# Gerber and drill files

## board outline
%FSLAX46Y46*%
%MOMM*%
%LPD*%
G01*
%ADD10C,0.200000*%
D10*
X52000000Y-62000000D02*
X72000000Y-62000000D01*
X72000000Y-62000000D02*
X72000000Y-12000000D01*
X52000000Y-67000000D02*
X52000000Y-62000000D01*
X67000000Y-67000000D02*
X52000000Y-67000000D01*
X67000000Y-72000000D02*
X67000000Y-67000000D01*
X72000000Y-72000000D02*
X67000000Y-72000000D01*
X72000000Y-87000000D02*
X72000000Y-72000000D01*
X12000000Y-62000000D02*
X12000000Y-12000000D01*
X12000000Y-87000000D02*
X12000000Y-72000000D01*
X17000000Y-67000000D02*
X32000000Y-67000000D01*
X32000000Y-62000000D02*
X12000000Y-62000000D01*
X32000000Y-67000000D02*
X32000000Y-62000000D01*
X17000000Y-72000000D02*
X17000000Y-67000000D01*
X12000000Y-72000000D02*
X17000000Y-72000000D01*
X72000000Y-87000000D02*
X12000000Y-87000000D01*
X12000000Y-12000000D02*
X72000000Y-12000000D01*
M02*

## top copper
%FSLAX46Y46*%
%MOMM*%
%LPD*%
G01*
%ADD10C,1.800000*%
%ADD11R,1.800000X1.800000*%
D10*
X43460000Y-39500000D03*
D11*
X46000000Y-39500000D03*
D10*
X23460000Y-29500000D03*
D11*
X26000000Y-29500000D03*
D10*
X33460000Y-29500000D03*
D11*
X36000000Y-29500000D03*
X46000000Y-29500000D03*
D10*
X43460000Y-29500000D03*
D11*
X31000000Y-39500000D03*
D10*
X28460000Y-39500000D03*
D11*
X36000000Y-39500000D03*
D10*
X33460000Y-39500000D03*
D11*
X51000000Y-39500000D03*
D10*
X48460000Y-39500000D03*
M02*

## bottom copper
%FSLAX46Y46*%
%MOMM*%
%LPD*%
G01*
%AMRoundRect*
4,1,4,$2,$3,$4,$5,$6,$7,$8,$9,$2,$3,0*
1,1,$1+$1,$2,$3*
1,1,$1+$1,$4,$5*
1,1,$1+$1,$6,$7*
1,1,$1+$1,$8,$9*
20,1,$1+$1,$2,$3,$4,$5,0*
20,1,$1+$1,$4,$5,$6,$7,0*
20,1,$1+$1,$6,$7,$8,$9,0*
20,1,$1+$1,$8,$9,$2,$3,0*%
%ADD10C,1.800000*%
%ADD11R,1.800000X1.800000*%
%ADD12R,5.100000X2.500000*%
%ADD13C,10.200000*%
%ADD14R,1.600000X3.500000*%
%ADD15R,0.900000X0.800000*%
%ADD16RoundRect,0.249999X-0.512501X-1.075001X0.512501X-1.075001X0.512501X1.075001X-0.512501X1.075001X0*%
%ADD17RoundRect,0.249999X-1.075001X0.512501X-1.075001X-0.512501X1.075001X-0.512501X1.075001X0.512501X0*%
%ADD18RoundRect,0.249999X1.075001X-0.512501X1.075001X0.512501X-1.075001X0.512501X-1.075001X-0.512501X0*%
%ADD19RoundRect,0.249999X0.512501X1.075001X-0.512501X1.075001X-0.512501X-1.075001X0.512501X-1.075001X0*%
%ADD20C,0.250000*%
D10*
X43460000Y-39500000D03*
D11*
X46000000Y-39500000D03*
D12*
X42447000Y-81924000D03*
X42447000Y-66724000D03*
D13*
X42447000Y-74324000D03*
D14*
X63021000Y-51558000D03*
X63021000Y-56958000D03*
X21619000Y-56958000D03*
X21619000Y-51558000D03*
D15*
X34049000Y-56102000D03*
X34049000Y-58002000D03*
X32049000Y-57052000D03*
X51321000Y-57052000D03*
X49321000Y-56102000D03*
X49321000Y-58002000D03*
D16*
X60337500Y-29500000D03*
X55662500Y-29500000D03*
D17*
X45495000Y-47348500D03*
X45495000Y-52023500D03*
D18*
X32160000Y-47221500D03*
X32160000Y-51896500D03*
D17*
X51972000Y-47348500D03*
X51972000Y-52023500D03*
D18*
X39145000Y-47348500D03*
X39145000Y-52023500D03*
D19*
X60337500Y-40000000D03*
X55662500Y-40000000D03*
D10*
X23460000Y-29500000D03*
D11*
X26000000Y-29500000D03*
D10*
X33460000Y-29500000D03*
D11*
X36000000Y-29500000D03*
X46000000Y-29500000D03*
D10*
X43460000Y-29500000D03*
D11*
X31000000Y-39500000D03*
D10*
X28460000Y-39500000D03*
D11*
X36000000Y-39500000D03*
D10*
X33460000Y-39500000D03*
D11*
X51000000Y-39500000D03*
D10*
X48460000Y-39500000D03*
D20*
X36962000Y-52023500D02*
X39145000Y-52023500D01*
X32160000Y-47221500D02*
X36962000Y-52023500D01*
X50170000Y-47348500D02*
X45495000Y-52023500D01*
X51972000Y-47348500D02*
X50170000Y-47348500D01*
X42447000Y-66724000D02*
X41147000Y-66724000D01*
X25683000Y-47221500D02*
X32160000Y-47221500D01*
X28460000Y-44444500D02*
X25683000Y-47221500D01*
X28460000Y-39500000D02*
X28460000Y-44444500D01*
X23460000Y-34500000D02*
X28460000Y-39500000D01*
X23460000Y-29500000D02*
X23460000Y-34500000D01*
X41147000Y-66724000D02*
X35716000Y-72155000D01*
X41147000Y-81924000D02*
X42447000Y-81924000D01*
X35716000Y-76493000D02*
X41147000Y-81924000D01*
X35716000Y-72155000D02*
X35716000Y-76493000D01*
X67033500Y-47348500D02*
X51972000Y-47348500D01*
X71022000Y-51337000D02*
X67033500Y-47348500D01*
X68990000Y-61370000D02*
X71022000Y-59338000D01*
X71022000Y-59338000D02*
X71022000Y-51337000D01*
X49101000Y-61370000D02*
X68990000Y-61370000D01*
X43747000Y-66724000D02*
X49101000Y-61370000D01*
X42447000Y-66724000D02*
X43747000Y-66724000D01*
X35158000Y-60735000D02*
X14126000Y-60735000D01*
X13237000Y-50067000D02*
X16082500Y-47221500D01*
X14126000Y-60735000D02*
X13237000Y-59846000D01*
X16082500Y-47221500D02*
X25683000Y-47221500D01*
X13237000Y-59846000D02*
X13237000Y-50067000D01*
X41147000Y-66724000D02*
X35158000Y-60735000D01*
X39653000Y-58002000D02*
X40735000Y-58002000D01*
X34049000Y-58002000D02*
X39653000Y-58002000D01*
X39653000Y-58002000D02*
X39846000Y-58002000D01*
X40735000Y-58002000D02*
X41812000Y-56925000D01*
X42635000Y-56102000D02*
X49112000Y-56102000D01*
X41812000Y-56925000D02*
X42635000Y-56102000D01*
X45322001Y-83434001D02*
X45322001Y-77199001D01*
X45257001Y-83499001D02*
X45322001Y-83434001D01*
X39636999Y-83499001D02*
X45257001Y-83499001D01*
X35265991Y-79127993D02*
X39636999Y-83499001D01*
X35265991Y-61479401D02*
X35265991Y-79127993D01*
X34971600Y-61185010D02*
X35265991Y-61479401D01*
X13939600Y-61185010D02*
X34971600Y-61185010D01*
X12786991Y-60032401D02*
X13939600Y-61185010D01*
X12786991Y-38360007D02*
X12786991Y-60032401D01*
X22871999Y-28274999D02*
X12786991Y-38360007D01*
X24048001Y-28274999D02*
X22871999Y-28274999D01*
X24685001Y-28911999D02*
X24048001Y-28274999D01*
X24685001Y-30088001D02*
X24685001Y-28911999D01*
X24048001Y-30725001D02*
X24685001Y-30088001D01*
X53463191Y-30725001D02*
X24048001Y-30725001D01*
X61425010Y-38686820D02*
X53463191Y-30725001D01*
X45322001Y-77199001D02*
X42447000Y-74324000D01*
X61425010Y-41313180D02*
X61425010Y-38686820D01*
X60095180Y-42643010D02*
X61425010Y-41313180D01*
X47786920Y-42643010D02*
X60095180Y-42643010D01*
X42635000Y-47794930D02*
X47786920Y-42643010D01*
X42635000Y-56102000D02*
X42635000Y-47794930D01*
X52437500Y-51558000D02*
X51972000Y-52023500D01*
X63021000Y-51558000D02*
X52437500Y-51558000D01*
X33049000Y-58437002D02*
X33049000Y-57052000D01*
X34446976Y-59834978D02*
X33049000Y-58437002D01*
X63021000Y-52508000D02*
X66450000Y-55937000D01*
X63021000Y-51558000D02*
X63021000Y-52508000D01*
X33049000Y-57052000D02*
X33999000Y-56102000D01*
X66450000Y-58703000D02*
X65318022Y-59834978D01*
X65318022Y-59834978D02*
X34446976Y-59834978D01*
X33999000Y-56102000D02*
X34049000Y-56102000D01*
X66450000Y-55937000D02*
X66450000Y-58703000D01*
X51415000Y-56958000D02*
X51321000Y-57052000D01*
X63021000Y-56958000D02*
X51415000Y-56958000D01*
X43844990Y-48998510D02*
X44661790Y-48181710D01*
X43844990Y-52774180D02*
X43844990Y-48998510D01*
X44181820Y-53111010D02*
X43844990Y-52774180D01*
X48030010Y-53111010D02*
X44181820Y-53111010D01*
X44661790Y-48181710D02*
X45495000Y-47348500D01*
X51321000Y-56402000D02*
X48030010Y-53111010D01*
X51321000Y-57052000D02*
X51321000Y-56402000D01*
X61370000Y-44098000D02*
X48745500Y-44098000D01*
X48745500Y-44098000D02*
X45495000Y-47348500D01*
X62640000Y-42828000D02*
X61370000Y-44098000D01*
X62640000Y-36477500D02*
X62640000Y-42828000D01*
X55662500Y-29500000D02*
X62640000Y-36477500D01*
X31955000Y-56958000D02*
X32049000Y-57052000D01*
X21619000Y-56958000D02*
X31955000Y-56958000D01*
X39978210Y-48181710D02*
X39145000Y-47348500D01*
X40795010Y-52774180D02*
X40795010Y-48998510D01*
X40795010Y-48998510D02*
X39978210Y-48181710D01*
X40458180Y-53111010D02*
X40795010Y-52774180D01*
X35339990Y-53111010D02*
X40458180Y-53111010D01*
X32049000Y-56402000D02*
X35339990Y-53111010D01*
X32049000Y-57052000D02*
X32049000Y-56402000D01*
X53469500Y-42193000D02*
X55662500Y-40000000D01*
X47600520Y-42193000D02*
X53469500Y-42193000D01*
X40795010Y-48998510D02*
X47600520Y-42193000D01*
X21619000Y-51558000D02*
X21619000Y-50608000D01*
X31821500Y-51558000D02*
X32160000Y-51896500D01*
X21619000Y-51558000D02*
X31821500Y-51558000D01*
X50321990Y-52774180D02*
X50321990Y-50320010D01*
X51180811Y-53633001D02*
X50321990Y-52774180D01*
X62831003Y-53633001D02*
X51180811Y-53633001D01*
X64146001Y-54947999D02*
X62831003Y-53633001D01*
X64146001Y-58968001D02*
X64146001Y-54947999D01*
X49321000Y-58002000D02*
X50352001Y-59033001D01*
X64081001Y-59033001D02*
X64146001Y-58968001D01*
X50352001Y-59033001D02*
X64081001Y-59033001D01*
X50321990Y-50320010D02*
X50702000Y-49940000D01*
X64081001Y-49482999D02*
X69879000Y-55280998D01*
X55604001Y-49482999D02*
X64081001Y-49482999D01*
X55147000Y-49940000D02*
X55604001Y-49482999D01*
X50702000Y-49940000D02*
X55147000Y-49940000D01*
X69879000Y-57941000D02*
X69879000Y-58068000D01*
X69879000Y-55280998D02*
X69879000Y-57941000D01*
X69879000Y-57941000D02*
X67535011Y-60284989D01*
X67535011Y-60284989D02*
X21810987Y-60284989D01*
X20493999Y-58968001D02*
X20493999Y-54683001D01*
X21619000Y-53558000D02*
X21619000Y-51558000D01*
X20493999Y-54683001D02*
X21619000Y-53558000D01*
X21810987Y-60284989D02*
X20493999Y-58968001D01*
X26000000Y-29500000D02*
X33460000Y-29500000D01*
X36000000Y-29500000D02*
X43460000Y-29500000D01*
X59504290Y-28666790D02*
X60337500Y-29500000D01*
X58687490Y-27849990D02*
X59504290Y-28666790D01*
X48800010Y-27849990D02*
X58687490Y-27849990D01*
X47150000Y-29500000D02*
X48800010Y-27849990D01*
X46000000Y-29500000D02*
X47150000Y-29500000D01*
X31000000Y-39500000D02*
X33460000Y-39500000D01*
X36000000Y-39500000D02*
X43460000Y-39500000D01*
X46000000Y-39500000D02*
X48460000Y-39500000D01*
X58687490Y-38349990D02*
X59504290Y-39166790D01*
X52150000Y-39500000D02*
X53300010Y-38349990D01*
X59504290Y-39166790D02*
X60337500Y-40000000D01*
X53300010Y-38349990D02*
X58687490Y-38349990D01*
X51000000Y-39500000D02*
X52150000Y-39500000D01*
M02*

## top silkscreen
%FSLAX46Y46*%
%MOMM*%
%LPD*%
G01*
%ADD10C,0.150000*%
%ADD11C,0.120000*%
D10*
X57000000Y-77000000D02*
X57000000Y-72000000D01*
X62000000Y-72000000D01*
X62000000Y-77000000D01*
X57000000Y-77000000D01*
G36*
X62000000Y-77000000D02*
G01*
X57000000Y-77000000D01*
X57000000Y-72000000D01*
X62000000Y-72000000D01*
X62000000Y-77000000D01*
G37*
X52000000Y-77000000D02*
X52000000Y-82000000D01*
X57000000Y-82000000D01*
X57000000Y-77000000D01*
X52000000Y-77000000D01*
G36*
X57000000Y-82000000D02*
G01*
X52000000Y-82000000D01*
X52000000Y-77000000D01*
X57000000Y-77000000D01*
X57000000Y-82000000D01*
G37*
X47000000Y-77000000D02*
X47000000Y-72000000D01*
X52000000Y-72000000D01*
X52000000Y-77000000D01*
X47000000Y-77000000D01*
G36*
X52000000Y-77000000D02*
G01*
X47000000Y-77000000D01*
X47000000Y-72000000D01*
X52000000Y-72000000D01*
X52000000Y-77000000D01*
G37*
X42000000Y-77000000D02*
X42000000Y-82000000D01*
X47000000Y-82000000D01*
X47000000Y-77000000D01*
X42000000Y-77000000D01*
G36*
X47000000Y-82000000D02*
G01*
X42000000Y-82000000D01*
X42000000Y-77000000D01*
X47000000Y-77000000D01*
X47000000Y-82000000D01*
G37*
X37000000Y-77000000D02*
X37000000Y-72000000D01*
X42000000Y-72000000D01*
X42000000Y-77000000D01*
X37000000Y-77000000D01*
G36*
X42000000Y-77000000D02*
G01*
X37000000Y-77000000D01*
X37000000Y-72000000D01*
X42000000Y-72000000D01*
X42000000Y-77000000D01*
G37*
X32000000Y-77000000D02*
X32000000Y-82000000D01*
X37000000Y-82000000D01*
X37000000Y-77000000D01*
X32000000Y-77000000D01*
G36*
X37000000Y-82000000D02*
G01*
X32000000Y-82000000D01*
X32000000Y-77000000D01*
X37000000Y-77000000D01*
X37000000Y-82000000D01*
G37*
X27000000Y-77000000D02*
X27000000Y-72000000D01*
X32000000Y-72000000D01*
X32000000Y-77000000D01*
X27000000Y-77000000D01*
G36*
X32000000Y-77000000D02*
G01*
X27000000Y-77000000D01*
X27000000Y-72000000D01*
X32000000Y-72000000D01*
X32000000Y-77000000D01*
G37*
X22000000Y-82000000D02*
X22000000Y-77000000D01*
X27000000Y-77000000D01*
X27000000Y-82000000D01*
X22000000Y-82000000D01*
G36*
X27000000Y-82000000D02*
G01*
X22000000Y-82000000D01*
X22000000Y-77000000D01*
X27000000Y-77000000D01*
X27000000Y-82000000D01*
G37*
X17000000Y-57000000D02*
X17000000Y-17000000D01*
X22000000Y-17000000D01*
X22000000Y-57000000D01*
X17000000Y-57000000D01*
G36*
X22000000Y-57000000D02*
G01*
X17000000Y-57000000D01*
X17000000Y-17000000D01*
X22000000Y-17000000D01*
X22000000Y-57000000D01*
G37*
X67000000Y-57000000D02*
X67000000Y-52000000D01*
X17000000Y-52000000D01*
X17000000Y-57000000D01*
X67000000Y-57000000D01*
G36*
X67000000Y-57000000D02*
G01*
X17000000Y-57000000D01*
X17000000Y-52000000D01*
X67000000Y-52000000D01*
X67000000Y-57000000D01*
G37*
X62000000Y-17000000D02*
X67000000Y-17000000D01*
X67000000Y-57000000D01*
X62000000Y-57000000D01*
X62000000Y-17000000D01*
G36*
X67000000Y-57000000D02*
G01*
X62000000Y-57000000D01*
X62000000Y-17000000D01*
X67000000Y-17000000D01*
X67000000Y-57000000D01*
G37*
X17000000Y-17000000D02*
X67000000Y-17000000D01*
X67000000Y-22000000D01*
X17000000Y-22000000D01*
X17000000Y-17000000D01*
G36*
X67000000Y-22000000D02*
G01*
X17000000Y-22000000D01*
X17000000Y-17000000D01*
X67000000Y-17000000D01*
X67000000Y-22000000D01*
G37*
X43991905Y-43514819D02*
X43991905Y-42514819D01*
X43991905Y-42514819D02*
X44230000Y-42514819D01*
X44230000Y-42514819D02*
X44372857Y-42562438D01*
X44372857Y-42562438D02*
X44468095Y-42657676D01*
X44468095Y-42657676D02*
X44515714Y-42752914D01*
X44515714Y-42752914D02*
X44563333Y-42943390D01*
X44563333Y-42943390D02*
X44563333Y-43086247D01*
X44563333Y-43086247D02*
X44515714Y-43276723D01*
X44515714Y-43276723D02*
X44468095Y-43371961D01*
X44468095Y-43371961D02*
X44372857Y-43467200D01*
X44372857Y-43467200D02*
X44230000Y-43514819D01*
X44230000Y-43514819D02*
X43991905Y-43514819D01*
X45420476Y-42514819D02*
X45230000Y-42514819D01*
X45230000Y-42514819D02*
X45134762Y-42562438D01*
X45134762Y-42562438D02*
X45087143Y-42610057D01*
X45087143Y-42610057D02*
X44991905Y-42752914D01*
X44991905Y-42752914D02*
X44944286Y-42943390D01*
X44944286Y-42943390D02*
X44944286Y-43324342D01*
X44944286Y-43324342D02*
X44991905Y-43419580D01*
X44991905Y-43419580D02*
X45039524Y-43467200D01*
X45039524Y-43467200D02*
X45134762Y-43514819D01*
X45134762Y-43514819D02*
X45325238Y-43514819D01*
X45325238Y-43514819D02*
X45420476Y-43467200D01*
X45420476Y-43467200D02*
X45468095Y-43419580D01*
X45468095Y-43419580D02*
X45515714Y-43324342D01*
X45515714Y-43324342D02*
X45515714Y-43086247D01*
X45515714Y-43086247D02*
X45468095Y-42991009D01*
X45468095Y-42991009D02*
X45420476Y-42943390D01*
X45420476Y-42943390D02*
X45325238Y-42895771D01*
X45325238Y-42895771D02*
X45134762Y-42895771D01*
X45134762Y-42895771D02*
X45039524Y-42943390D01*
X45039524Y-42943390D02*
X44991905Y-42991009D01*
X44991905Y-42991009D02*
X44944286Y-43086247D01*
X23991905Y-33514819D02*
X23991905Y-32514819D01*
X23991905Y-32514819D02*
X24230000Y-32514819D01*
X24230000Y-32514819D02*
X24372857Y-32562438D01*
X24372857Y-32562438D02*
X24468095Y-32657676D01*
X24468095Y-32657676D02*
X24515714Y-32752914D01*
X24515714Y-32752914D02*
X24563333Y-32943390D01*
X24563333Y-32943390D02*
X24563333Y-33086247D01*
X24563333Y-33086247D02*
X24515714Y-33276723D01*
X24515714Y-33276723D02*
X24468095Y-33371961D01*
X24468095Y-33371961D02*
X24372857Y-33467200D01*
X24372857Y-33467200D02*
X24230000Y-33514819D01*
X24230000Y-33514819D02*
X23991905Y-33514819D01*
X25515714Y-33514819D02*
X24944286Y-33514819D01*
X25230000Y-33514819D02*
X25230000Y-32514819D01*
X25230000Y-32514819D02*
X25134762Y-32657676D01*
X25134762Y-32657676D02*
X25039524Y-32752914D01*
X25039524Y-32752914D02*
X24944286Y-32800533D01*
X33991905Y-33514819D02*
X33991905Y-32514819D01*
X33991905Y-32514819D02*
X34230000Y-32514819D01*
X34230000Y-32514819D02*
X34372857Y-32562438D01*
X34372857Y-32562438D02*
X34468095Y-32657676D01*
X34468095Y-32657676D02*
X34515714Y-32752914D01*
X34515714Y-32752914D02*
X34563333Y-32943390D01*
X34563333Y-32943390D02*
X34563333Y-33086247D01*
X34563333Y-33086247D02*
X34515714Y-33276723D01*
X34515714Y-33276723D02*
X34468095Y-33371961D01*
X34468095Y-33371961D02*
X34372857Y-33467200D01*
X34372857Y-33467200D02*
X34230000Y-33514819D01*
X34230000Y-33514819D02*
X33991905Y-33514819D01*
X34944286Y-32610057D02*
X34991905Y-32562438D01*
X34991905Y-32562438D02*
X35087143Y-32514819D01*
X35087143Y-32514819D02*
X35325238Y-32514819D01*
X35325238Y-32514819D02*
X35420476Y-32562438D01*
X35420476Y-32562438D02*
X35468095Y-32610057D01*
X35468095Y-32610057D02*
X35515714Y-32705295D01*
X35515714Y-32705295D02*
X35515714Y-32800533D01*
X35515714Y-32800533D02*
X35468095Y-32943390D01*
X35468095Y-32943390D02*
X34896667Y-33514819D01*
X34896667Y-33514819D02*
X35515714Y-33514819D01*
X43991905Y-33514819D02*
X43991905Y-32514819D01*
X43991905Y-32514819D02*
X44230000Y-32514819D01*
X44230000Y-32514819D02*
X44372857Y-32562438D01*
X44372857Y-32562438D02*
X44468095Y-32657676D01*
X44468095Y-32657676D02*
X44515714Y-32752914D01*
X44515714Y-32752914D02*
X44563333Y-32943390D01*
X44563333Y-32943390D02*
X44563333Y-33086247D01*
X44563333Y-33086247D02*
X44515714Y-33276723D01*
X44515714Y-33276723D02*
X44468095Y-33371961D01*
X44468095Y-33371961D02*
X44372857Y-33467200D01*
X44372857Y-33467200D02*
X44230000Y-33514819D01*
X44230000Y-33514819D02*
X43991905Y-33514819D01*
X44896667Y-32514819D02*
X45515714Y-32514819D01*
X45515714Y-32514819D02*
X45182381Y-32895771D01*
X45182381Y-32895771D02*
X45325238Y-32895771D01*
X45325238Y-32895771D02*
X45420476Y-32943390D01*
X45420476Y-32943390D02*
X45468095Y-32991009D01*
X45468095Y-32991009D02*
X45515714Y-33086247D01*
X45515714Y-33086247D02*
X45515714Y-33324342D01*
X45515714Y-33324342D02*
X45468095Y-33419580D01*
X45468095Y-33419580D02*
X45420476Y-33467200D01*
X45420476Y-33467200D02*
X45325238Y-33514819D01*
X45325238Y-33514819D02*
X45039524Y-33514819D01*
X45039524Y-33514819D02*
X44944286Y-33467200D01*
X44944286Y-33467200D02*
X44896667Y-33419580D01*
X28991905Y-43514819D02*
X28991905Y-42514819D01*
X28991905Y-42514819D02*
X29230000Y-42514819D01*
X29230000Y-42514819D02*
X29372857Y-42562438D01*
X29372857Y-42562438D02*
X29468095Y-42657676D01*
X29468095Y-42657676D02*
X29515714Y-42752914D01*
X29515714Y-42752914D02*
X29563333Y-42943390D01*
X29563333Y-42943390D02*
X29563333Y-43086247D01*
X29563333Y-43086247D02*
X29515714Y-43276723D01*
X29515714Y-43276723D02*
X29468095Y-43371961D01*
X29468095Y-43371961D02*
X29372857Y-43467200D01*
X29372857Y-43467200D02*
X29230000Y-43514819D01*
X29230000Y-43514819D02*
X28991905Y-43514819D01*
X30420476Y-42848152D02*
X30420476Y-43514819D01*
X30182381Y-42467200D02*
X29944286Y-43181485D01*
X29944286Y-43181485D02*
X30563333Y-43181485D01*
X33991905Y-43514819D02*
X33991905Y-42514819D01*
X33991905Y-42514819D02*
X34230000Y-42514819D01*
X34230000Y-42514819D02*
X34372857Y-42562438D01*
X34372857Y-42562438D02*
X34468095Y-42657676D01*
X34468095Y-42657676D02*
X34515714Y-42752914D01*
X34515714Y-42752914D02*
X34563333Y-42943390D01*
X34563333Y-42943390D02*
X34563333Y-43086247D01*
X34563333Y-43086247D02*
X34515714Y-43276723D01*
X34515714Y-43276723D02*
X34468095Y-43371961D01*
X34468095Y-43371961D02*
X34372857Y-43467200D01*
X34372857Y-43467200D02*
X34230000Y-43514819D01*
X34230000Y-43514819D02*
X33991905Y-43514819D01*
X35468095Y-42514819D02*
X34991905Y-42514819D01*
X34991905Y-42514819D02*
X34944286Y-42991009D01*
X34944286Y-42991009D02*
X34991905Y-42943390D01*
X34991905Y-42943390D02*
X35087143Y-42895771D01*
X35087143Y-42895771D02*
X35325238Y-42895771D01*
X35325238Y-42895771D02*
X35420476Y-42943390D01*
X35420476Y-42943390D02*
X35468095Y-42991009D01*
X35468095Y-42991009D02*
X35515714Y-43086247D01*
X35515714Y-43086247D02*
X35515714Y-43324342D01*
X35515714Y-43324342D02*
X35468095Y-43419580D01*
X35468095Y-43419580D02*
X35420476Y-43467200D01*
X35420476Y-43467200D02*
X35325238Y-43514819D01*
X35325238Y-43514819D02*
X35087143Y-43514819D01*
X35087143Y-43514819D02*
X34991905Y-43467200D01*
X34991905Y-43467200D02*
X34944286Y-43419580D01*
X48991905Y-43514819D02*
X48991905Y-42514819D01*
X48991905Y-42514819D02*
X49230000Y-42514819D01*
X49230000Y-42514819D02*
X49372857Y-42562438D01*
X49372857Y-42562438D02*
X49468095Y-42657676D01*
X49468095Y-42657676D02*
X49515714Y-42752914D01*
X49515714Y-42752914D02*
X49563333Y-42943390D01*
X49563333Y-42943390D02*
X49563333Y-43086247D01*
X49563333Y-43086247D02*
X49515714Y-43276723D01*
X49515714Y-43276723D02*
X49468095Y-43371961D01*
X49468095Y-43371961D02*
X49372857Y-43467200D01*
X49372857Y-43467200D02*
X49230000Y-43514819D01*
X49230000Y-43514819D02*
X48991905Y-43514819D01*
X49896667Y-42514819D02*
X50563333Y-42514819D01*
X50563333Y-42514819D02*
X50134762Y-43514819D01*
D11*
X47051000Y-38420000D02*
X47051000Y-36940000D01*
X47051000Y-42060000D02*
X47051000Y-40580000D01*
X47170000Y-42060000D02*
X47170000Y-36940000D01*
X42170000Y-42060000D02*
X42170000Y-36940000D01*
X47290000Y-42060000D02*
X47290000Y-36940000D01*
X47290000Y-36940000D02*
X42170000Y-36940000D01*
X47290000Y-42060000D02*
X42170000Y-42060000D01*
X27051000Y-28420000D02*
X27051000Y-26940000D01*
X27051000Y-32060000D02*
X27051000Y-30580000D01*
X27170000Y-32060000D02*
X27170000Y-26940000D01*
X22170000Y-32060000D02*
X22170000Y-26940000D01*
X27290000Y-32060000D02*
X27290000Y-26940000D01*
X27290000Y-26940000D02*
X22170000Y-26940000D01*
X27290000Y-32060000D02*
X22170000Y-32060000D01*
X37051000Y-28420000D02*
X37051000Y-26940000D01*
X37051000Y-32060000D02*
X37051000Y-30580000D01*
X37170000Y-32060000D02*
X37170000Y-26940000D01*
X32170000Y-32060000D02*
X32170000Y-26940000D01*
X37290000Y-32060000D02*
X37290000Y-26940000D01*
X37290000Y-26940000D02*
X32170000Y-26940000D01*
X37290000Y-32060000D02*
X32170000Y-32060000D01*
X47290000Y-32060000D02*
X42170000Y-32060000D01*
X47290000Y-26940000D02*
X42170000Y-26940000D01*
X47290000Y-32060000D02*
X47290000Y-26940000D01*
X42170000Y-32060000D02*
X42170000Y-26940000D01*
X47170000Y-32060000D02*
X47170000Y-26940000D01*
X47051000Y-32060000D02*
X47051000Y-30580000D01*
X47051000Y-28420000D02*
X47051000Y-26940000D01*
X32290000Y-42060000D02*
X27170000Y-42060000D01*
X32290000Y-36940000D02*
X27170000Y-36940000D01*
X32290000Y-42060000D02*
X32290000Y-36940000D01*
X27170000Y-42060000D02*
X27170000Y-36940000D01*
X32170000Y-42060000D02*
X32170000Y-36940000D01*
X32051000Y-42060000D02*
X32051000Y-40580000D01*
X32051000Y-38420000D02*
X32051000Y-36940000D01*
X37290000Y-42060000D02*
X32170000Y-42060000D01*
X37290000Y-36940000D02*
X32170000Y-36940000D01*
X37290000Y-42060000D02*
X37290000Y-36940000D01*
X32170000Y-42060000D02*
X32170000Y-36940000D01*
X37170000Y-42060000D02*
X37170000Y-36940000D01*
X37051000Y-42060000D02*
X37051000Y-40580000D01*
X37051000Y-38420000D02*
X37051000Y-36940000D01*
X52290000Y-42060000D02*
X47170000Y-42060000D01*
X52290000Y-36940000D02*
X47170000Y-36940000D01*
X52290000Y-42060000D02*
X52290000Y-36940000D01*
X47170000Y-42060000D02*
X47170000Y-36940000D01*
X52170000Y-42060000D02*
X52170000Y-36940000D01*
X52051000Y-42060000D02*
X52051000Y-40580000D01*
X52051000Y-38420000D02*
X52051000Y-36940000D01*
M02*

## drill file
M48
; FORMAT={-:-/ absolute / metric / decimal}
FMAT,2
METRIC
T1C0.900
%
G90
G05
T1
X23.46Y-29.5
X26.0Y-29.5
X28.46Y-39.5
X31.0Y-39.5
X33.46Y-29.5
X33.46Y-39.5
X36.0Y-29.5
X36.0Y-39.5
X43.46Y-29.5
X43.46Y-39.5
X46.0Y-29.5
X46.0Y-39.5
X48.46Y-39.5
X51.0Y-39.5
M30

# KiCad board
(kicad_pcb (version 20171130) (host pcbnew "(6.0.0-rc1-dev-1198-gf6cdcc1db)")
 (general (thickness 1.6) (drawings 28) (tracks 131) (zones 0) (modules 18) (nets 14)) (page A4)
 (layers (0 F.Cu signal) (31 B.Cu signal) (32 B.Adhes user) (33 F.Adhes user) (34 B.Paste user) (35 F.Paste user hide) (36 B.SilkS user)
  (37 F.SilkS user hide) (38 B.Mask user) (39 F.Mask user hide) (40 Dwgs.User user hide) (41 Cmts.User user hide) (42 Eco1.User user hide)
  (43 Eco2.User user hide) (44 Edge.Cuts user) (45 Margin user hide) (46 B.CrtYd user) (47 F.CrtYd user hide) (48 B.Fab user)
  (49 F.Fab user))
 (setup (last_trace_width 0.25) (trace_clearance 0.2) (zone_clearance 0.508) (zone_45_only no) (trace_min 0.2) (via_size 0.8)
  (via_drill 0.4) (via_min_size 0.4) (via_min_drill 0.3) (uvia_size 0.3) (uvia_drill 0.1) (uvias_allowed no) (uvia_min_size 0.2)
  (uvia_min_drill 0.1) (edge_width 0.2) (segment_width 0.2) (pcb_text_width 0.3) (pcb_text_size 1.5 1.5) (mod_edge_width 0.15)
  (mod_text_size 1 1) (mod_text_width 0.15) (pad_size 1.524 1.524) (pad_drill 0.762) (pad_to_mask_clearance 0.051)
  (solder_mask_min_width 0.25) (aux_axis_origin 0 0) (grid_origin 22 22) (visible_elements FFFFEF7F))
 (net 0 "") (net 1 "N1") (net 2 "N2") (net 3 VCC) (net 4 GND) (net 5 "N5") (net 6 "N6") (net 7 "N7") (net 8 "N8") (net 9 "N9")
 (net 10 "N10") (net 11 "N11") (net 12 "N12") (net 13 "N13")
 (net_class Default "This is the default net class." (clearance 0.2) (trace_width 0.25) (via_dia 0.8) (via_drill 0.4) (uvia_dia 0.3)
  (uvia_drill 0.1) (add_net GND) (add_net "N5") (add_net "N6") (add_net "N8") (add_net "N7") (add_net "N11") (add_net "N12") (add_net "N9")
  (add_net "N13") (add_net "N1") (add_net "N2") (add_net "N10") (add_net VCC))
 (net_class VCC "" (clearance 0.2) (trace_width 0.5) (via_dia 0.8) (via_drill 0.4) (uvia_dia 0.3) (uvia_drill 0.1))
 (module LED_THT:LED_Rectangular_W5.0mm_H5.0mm (layer F.Cu) (at 46 39.5 180)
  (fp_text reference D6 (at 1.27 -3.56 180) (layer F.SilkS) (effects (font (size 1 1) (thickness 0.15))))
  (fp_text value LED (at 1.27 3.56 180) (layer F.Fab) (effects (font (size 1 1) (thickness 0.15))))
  (fp_line (start -1.051 1.08) (end -1.051 2.56) (layer F.SilkS) (width 0.12))
  (fp_line (start -1.051 -2.56) (end -1.051 -1.08) (layer F.SilkS) (width 0.12))
  (fp_line (start -1.17 -2.56) (end -1.17 2.56) (layer F.SilkS) (width 0.12))
  (fp_line (start 3.83 -2.56) (end 3.83 2.56) (layer F.SilkS) (width 0.12))
  (fp_line (start -1.29 -2.56) (end -1.29 2.56) (layer F.SilkS) (width 0.12))
  (fp_line (start -1.29 2.56) (end 3.83 2.56) (layer F.SilkS) (width 0.12))
  (fp_line (start -1.29 -2.56) (end 3.83 -2.56) (layer F.SilkS) (width 0.12))
  (pad 2 thru_hole circle (at 2.54 0 180) (size 1.8 1.8) (drill 0.9) (layers *.Cu *.Mask) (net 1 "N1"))
  (pad 1 thru_hole rect (at 0 0 180) (size 1.8 1.8) (drill 0.9) (layers *.Cu *.Mask) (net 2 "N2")))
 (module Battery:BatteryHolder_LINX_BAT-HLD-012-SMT (layer B.Cu) (at 42.447 74.324 90)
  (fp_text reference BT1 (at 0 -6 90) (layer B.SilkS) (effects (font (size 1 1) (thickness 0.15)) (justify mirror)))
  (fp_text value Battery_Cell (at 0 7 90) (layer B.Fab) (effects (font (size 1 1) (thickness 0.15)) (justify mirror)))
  (pad 1 smd rect (at -7.6 0 90) (size 2.5 5.1) (layers B.Cu B.Paste B.Mask) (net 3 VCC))
  (pad 1 smd rect (at 7.6 0 90) (size 2.5 5.1) (layers B.Cu B.Paste B.Mask) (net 3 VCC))
  (pad 2 smd circle (at 0 0 90) (size 10.2 10.2) (layers B.Cu B.Paste B.Mask) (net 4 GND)))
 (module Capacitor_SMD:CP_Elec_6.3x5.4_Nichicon (layer B.Cu) (at 63.021 54.258 270)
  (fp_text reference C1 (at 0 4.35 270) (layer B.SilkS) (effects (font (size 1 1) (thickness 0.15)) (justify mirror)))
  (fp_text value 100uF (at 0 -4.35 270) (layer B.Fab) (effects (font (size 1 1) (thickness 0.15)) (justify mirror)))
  (pad 1 smd rect (at -2.7 0 270) (size 3.5 1.6) (layers B.Cu B.Paste B.Mask) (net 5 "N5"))
  (pad 2 smd rect (at 2.7 0 270) (size 3.5 1.6) (layers B.Cu B.Paste B.Mask) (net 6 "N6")))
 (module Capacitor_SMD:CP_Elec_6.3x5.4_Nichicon (layer B.Cu) (at 21.619 54.258 270)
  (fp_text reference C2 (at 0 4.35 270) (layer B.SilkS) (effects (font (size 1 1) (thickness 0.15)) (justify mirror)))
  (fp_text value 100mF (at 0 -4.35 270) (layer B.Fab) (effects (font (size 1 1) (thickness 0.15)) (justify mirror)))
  (pad 2 smd rect (at 2.7 0 270) (size 3.5 1.6) (layers B.Cu B.Paste B.Mask) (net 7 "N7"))
  (pad 1 smd rect (at -2.7 0 270) (size 3.5 1.6) (layers B.Cu B.Paste B.Mask) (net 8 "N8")))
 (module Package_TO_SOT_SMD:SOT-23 (layer B.Cu) (at 33.049 57.052 180)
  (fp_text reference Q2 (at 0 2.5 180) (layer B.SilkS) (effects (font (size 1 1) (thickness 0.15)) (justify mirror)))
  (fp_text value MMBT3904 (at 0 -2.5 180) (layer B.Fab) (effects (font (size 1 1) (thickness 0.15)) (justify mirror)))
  (pad 1 smd rect (at -1 0.95 180) (size 0.9 0.8) (layers B.Cu B.Paste B.Mask) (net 5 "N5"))
  (pad 2 smd rect (at -1 -0.95 180) (size 0.9 0.8) (layers B.Cu B.Paste B.Mask) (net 4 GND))
  (pad 3 smd rect (at 1 0 180) (size 0.9 0.8) (layers B.Cu B.Paste B.Mask) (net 7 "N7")))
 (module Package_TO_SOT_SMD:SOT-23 (layer B.Cu) (at 50.321 57.052)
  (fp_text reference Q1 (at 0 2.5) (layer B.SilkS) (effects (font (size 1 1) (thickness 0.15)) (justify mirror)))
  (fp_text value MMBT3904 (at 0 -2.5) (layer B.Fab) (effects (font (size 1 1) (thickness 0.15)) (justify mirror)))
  (pad 3 smd rect (at 1 0) (size 0.9 0.8) (layers B.Cu B.Paste B.Mask) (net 6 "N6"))
  (pad 2 smd rect (at -1 -0.95) (size 0.9 0.8) (layers B.Cu B.Paste B.Mask) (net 4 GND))
  (pad 1 smd rect (at -1 0.95) (size 0.9 0.8) (layers B.Cu B.Paste B.Mask) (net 8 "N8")))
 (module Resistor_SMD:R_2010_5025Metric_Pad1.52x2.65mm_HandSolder (layer B.Cu) (at 58 29.5)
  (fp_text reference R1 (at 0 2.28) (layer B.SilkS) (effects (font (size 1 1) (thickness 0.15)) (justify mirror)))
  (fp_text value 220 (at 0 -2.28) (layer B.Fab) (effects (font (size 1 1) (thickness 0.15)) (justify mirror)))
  (pad 2 smd roundrect (at 2.3375 0) (size 1.525 2.65) (layers B.Cu B.Paste B.Mask) (roundrect_rratio 0.163934) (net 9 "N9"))
  (pad 1 smd roundrect (at -2.3375 0) (size 1.525 2.65) (layers B.Cu B.Paste B.Mask) (roundrect_rratio 0.163934) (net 6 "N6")))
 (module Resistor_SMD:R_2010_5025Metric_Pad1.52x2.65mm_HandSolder (layer B.Cu) (at 45.495 49.686 270)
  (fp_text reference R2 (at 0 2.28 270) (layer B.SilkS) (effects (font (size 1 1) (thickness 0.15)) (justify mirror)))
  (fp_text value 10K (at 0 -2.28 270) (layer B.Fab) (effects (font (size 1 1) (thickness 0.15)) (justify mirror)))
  (pad 1 smd roundrect (at -2.3375 0 270) (size 1.525 2.65) (layers B.Cu B.Paste B.Mask) (roundrect_rratio 0.163934) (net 6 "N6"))
  (pad 2 smd roundrect (at 2.3375 0 270) (size 1.525 2.65) (layers B.Cu B.Paste B.Mask) (roundrect_rratio 0.163934) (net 3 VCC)))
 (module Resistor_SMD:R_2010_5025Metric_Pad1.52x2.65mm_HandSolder (layer B.Cu) (at 32.16 49.559 90)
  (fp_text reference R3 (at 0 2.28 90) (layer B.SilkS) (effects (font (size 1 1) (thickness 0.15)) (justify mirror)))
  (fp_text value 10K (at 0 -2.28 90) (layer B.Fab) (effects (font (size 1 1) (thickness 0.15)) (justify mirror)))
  (pad 2 smd roundrect (at 2.3375 0 90) (size 1.525 2.65) (layers B.Cu B.Paste B.Mask) (roundrect_rratio 0.163934) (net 3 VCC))
  (pad 1 smd roundrect (at -2.3375 0 90) (size 1.525 2.65) (layers B.Cu B.Paste B.Mask) (roundrect_rratio 0.163934) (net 8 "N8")))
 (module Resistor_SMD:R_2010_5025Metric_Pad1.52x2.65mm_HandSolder (layer B.Cu) (at 51.972 49.686 270)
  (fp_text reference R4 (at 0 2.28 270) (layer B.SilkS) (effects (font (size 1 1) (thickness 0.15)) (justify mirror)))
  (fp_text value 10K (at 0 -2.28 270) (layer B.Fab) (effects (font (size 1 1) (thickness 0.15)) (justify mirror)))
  (pad 1 smd roundrect (at -2.3375 0 270) (size 1.525 2.65) (layers B.Cu B.Paste B.Mask) (roundrect_rratio 0.163934) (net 3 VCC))
  (pad 2 smd roundrect (at 2.3375 0 270) (size 1.525 2.65) (layers B.Cu B.Paste B.Mask) (roundrect_rratio 0.163934) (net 5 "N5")))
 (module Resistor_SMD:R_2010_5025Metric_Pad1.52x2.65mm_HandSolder (layer B.Cu) (at 39.145 49.686 90)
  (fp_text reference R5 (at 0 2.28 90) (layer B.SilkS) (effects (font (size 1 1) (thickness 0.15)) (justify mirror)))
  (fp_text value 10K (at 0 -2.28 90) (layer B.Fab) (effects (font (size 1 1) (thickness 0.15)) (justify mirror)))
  (pad 2 smd roundrect (at 2.3375 0 90) (size 1.525 2.65) (layers B.Cu B.Paste B.Mask) (roundrect_rratio 0.163934) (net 7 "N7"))
  (pad 1 smd roundrect (at -2.3375 0 90) (size 1.525 2.65) (layers B.Cu B.Paste B.Mask) (roundrect_rratio 0.163934) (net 3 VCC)))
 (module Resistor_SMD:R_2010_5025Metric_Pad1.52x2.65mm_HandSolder (layer B.Cu) (at 58 40 180)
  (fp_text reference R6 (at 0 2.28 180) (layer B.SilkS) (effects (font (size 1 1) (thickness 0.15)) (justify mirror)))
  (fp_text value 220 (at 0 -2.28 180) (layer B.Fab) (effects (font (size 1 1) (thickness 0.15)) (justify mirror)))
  (pad 1 smd roundrect (at -2.3375 0 180) (size 1.525 2.65) (layers B.Cu B.Paste B.Mask) (roundrect_rratio 0.163934) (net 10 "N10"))
  (pad 2 smd roundrect (at 2.3375 0 180) (size 1.525 2.65) (layers B.Cu B.Paste B.Mask) (roundrect_rratio 0.163934) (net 7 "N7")))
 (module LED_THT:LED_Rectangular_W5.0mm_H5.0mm (layer F.Cu) (at 26 29.5 180)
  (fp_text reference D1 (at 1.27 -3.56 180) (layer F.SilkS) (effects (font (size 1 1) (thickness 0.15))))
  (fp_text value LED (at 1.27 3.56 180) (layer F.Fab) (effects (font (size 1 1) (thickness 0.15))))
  (fp_line (start -1.051 1.08) (end -1.051 2.56) (layer F.SilkS) (width 0.12))
  (fp_line (start -1.051 -2.56) (end -1.051 -1.08) (layer F.SilkS) (width 0.12))
  (fp_line (start -1.17 -2.56) (end -1.17 2.56) (layer F.SilkS) (width 0.12))
  (fp_line (start 3.83 -2.56) (end 3.83 2.56) (layer F.SilkS) (width 0.12))
  (fp_line (start -1.29 -2.56) (end -1.29 2.56) (layer F.SilkS) (width 0.12))
  (fp_line (start -1.29 2.56) (end 3.83 2.56) (layer F.SilkS) (width 0.12))
  (fp_line (start -1.29 -2.56) (end 3.83 -2.56) (layer F.SilkS) (width 0.12))
  (pad 2 thru_hole circle (at 2.54 0 180) (size 1.8 1.8) (drill 0.9) (layers *.Cu *.Mask) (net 3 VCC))
  (pad 1 thru_hole rect (at 0 0 180) (size 1.8 1.8) (drill 0.9) (layers *.Cu *.Mask) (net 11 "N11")))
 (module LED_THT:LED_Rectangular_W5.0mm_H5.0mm (layer F.Cu) (at 36 29.5 180)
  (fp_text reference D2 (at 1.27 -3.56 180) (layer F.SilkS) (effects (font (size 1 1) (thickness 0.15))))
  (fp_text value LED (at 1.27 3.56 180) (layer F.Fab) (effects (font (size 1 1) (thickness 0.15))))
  (fp_line (start -1.051 1.08) (end -1.051 2.56) (layer F.SilkS) (width 0.12))
  (fp_line (start -1.051 -2.56) (end -1.051 -1.08) (layer F.SilkS) (width 0.12))
  (fp_line (start -1.17 -2.56) (end -1.17 2.56) (layer F.SilkS) (width 0.12))
  (fp_line (start 3.83 -2.56) (end 3.83 2.56) (layer F.SilkS) (width 0.12))
  (fp_line (start -1.29 -2.56) (end -1.29 2.56) (layer F.SilkS) (width 0.12))
  (fp_line (start -1.29 2.56) (end 3.83 2.56) (layer F.SilkS) (width 0.12))
  (fp_line (start -1.29 -2.56) (end 3.83 -2.56) (layer F.SilkS) (width 0.12))
  (pad 2 thru_hole circle (at 2.54 0 180) (size 1.8 1.8) (drill 0.9) (layers *.Cu *.Mask) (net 11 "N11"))
  (pad 1 thru_hole rect (at 0 0 180) (size 1.8 1.8) (drill 0.9) (layers *.Cu *.Mask) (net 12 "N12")))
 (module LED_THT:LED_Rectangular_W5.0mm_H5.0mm (layer F.Cu) (at 46 29.5 180)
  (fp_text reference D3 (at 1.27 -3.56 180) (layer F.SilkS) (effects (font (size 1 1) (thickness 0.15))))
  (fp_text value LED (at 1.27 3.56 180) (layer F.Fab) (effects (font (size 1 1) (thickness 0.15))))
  (fp_line (start -1.29 -2.56) (end 3.83 -2.56) (layer F.SilkS) (width 0.12))
  (fp_line (start -1.29 2.56) (end 3.83 2.56) (layer F.SilkS) (width 0.12))
  (fp_line (start -1.29 -2.56) (end -1.29 2.56) (layer F.SilkS) (width 0.12))
  (fp_line (start 3.83 -2.56) (end 3.83 2.56) (layer F.SilkS) (width 0.12))
  (fp_line (start -1.17 -2.56) (end -1.17 2.56) (layer F.SilkS) (width 0.12))
  (fp_line (start -1.051 -2.56) (end -1.051 -1.08) (layer F.SilkS) (width 0.12))
  (fp_line (start -1.051 1.08) (end -1.051 2.56) (layer F.SilkS) (width 0.12))
  (pad 1 thru_hole rect (at 0 0 180) (size 1.8 1.8) (drill 0.9) (layers *.Cu *.Mask) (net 9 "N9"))
  (pad 2 thru_hole circle (at 2.54 0 180) (size 1.8 1.8) (drill 0.9) (layers *.Cu *.Mask) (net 12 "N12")))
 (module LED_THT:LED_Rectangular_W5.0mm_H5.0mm (layer F.Cu) (at 31 39.5 180)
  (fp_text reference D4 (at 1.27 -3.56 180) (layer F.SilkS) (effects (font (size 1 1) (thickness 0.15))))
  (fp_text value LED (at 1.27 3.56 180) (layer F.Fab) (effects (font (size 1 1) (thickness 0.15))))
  (fp_line (start -1.29 -2.56) (end 3.83 -2.56) (layer F.SilkS) (width 0.12))
  (fp_line (start -1.29 2.56) (end 3.83 2.56) (layer F.SilkS) (width 0.12))
  (fp_line (start -1.29 -2.56) (end -1.29 2.56) (layer F.SilkS) (width 0.12))
  (fp_line (start 3.83 -2.56) (end 3.83 2.56) (layer F.SilkS) (width 0.12))
  (fp_line (start -1.17 -2.56) (end -1.17 2.56) (layer F.SilkS) (width 0.12))
  (fp_line (start -1.051 -2.56) (end -1.051 -1.08) (layer F.SilkS) (width 0.12))
  (fp_line (start -1.051 1.08) (end -1.051 2.56) (layer F.SilkS) (width 0.12))
  (pad 1 thru_hole rect (at 0 0 180) (size 1.8 1.8) (drill 0.9) (layers *.Cu *.Mask) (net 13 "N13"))
  (pad 2 thru_hole circle (at 2.54 0 180) (size 1.8 1.8) (drill 0.9) (layers *.Cu *.Mask) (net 3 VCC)))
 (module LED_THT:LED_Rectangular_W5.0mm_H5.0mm (layer F.Cu) (at 36 39.5 180)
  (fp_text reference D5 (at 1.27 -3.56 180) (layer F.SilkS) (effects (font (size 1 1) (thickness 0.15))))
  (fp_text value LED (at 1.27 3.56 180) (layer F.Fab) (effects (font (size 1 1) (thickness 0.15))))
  (fp_line (start -1.29 -2.56) (end 3.83 -2.56) (layer F.SilkS) (width 0.12))
  (fp_line (start -1.29 2.56) (end 3.83 2.56) (layer F.SilkS) (width 0.12))
  (fp_line (start -1.29 -2.56) (end -1.29 2.56) (layer F.SilkS) (width 0.12))
  (fp_line (start 3.83 -2.56) (end 3.83 2.56) (layer F.SilkS) (width 0.12))
  (fp_line (start -1.17 -2.56) (end -1.17 2.56) (layer F.SilkS) (width 0.12))
  (fp_line (start -1.051 -2.56) (end -1.051 -1.08) (layer F.SilkS) (width 0.12))
  (fp_line (start -1.051 1.08) (end -1.051 2.56) (layer F.SilkS) (width 0.12))
  (pad 1 thru_hole rect (at 0 0 180) (size 1.8 1.8) (drill 0.9) (layers *.Cu *.Mask) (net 1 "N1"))
  (pad 2 thru_hole circle (at 2.54 0 180) (size 1.8 1.8) (drill 0.9) (layers *.Cu *.Mask) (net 13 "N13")))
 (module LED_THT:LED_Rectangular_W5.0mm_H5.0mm (layer F.Cu) (at 51 39.5 180)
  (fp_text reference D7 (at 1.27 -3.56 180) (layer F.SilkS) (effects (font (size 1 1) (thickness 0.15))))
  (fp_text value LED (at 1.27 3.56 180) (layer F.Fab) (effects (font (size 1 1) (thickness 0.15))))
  (fp_line (start -1.29 -2.56) (end 3.83 -2.56) (layer F.SilkS) (width 0.12))
  (fp_line (start -1.29 2.56) (end 3.83 2.56) (layer F.SilkS) (width 0.12))
  (fp_line (start -1.29 -2.56) (end -1.29 2.56) (layer F.SilkS) (width 0.12))
  (fp_line (start 3.83 -2.56) (end 3.83 2.56) (layer F.SilkS) (width 0.12))
  (fp_line (start -1.17 -2.56) (end -1.17 2.56) (layer F.SilkS) (width 0.12))
  (fp_line (start -1.051 -2.56) (end -1.051 -1.08) (layer F.SilkS) (width 0.12))
  (fp_line (start -1.051 1.08) (end -1.051 2.56) (layer F.SilkS) (width 0.12))
  (pad 1 thru_hole rect (at 0 0 180) (size 1.8 1.8) (drill 0.9) (layers *.Cu *.Mask) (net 10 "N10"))
  (pad 2 thru_hole circle (at 2.54 0 180) (size 1.8 1.8) (drill 0.9) (layers *.Cu *.Mask) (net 2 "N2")))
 (gr_poly (pts (xy 57 77) (xy 57 72) (xy 62 72) (xy 62 77)) (layer F.SilkS) (width 0.15))
 (gr_poly (pts (xy 52 77) (xy 52 82) (xy 57 82) (xy 57 77)) (layer F.SilkS) (width 0.15))
 (gr_poly (pts (xy 47 77) (xy 47 72) (xy 52 72) (xy 52 77)) (layer F.SilkS) (width 0.15))
 (gr_poly (pts (xy 42 77) (xy 42 82) (xy 47 82) (xy 47 77)) (layer F.SilkS) (width 0.15))
 (gr_poly (pts (xy 37 77) (xy 37 72) (xy 42 72) (xy 42 77)) (layer F.SilkS) (width 0.15))
 (gr_poly (pts (xy 32 77) (xy 32 82) (xy 37 82) (xy 37 77)) (layer F.SilkS) (width 0.15))
 (gr_poly (pts (xy 27 77) (xy 27 72) (xy 32 72) (xy 32 77)) (layer F.SilkS) (width 0.15))
 (gr_poly (pts (xy 22 82) (xy 22 77) (xy 27 77) (xy 27 82)) (layer F.SilkS) (width 0.15))
 (gr_poly (pts (xy 17 57) (xy 17 17) (xy 22 17) (xy 22 57)) (layer F.SilkS) (width 0.15))
 (gr_poly (pts (xy 67 57) (xy 67 52) (xy 17 52) (xy 17 57)) (layer F.SilkS) (width 0.15))
 (gr_poly (pts (xy 62 17) (xy 67 17) (xy 67 57) (xy 62 57)) (layer F.SilkS) (width 0.15))
 (gr_poly (pts (xy 17 17) (xy 67 17) (xy 67 22) (xy 17 22)) (layer F.SilkS) (width 0.15))
 (gr_line (start 52 62) (end 72 62) (layer Edge.Cuts) (width 0.2))
 (gr_line (start 72 62) (end 72 12) (layer Edge.Cuts) (width 0.2))
 (gr_line (start 52 67) (end 52 62) (layer Edge.Cuts) (width 0.2))
 (gr_line (start 67 67) (end 52 67) (layer Edge.Cuts) (width 0.2))
 (gr_line (start 67 72) (end 67 67) (layer Edge.Cuts) (width 0.2))
 (gr_line (start 72 72) (end 67 72) (layer Edge.Cuts) (width 0.2))
 (gr_line (start 72 87) (end 72 72) (layer Edge.Cuts) (width 0.2))
 (gr_line (start 12 62) (end 12 12) (layer Edge.Cuts) (width 0.2))
 (gr_line (start 12 87) (end 12 72) (layer Edge.Cuts) (width 0.2))
 (gr_line (start 17 67) (end 32 67) (layer Edge.Cuts) (width 0.2))
 (gr_line (start 32 62) (end 12 62) (layer Edge.Cuts) (width 0.2))
 (gr_line (start 32 67) (end 32 62) (layer Edge.Cuts) (width 0.2))
 (gr_line (start 17 72) (end 17 67) (layer Edge.Cuts) (width 0.2))
 (gr_line (start 12 72) (end 17 72) (layer Edge.Cuts) (width 0.2))
 (gr_line (start 72 87) (end 12 87) (layer Edge.Cuts) (width 0.2))
 (gr_line (start 12 12) (end 72 12) (layer Edge.Cuts) (width 0.2))
 (segment (start 36.962 52.0235) (end 39.145 52.0235) (width 0.25) (layer B.Cu) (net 3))
 (segment (start 32.16 47.2215) (end 36.962 52.0235) (width 0.25) (layer B.Cu) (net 3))
 (segment (start 50.17 47.3485) (end 45.495 52.0235) (width 0.25) (layer B.Cu) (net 3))
 (segment (start 51.972 47.3485) (end 50.17 47.3485) (width 0.25) (layer B.Cu) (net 3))
 (segment (start 42.447 66.724) (end 41.147 66.724) (width 0.25) (layer B.Cu) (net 3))
 (segment (start 25.683 47.2215) (end 32.16 47.2215) (width 0.25) (layer B.Cu) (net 3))
 (segment (start 28.46 44.4445) (end 25.683 47.2215) (width 0.25) (layer B.Cu) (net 3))
 (segment (start 28.46 39.5) (end 28.46 44.4445) (width 0.25) (layer B.Cu) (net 3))
 (segment (start 23.46 34.5) (end 28.46 39.5) (width 0.25) (layer B.Cu) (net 3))
 (segment (start 23.46 29.5) (end 23.46 34.5) (width 0.25) (layer B.Cu) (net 3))
 (segment (start 41.147 66.724) (end 35.716 72.155) (width 0.25) (layer B.Cu) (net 3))
 (segment (start 41.147 81.924) (end 42.447 81.924) (width 0.25) (layer B.Cu) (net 3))
 (segment (start 35.716 76.493) (end 41.147 81.924) (width 0.25) (layer B.Cu) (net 3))
 (segment (start 35.716 72.155) (end 35.716 76.493) (width 0.25) (layer B.Cu) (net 3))
 (segment (start 67.0335 47.3485) (end 51.972 47.3485) (width 0.25) (layer B.Cu) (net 3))
 (segment (start 71.022 51.337) (end 67.0335 47.3485) (width 0.25) (layer B.Cu) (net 3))
 (segment (start 68.99 61.37) (end 71.022 59.338) (width 0.25) (layer B.Cu) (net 3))
 (segment (start 71.022 59.338) (end 71.022 51.337) (width 0.25) (layer B.Cu) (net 3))
 (segment (start 49.101 61.37) (end 68.99 61.37) (width 0.25) (layer B.Cu) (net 3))
 (segment (start 43.747 66.724) (end 49.101 61.37) (width 0.25) (layer B.Cu) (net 3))
 (segment (start 42.447 66.724) (end 43.747 66.724) (width 0.25) (layer B.Cu) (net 3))
 (segment (start 35.158 60.735) (end 14.126 60.735) (width 0.25) (layer B.Cu) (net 3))
 (segment (start 13.237 50.067) (end 16.0825 47.2215) (width 0.25) (layer B.Cu) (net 3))
 (segment (start 14.126 60.735) (end 13.237 59.846) (width 0.25) (layer B.Cu) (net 3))
 (segment (start 16.0825 47.2215) (end 25.683 47.2215) (width 0.25) (layer B.Cu) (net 3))
 (segment (start 13.237 59.846) (end 13.237 50.067) (width 0.25) (layer B.Cu) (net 3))
 (segment (start 41.147 66.724) (end 35.158 60.735) (width 0.25) (layer B.Cu) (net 3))
 (segment (start 39.653 58.002) (end 40.735 58.002) (width 0.25) (layer B.Cu) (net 4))
 (segment (start 34.049 58.002) (end 39.653 58.002) (width 0.25) (layer B.Cu) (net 4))
 (segment (start 39.653 58.002) (end 39.846 58.002) (width 0.25) (layer B.Cu) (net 4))
 (segment (start 40.735 58.002) (end 41.812 56.925) (width 0.25) (layer B.Cu) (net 4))
 (segment (start 42.635 56.102) (end 49.112 56.102) (width 0.25) (layer B.Cu) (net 4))
 (segment (start 41.812 56.925) (end 42.635 56.102) (width 0.25) (layer B.Cu) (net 4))
 (segment (start 45.322001 83.434001) (end 45.322001 77.199001) (width 0.25) (layer B.Cu) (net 4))
 (segment (start 45.257001 83.499001) (end 45.322001 83.434001) (width 0.25) (layer B.Cu) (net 4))
 (segment (start 39.636999 83.499001) (end 45.257001 83.499001) (width 0.25) (layer B.Cu) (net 4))
 (segment (start 35.265991 79.127993) (end 39.636999 83.499001) (width 0.25) (layer B.Cu) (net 4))
 (segment (start 35.265991 61.479401) (end 35.265991 79.127993) (width 0.25) (layer B.Cu) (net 4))
 (segment (start 34.9716 61.18501) (end 35.265991 61.479401) (width 0.25) (layer B.Cu) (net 4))
 (segment (start 13.9396 61.18501) (end 34.9716 61.18501) (width 0.25) (layer B.Cu) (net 4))
 (segment (start 12.786991 60.032401) (end 13.9396 61.18501) (width 0.25) (layer B.Cu) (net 4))
 (segment (start 12.786991 38.360007) (end 12.786991 60.032401) (width 0.25) (layer B.Cu) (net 4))
 (segment (start 22.871999 28.274999) (end 12.786991 38.360007) (width 0.25) (layer B.Cu) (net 4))
 (segment (start 24.048001 28.274999) (end 22.871999 28.274999) (width 0.25) (layer B.Cu) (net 4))
 (segment (start 24.685001 28.911999) (end 24.048001 28.274999) (width 0.25) (layer B.Cu) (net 4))
 (segment (start 24.685001 30.088001) (end 24.685001 28.911999) (width 0.25) (layer B.Cu) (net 4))
 (segment (start 24.048001 30.725001) (end 24.685001 30.088001) (width 0.25) (layer B.Cu) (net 4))
 (segment (start 53.463191 30.725001) (end 24.048001 30.725001) (width 0.25) (layer B.Cu) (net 4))
 (segment (start 61.42501 38.68682) (end 53.463191 30.725001) (width 0.25) (layer B.Cu) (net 4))
 (segment (start 45.322001 77.199001) (end 42.447 74.324) (width 0.25) (layer B.Cu) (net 4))
 (segment (start 61.42501 41.31318) (end 61.42501 38.68682) (width 0.25) (layer B.Cu) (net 4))
 (segment (start 60.09518 42.64301) (end 61.42501 41.31318) (width 0.25) (layer B.Cu) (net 4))
 (segment (start 47.78692 42.64301) (end 60.09518 42.64301) (width 0.25) (layer B.Cu) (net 4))
 (segment (start 42.635 47.79493) (end 47.78692 42.64301) (width 0.25) (layer B.Cu) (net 4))
 (segment (start 42.635 56.102) (end 42.635 47.79493) (width 0.25) (layer B.Cu) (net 4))
 (segment (start 52.4375 51.558) (end 51.972 52.0235) (width 0.25) (layer B.Cu) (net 5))
 (segment (start 63.021 51.558) (end 52.4375 51.558) (width 0.25) (layer B.Cu) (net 5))
 (segment (start 33.049 58.437002) (end 33.049 57.052) (width 0.25) (layer B.Cu) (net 5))
 (segment (start 34.446976 59.834978) (end 33.049 58.437002) (width 0.25) (layer B.Cu) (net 5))
 (segment (start 63.021 52.508) (end 66.45 55.937) (width 0.25) (layer B.Cu) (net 5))
 (segment (start 63.021 51.558) (end 63.021 52.508) (width 0.25) (layer B.Cu) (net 5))
 (segment (start 33.049 57.052) (end 33.999 56.102) (width 0.25) (layer B.Cu) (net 5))
 (segment (start 66.45 58.703) (end 65.318022 59.834978) (width 0.25) (layer B.Cu) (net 5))
 (segment (start 65.318022 59.834978) (end 34.446976 59.834978) (width 0.25) (layer B.Cu) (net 5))
 (segment (start 33.999 56.102) (end 34.049 56.102) (width 0.25) (layer B.Cu) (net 5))
 (segment (start 66.45 55.937) (end 66.45 58.703) (width 0.25) (layer B.Cu) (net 5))
 (segment (start 51.415 56.958) (end 51.321 57.052) (width 0.25) (layer B.Cu) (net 6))
 (segment (start 63.021 56.958) (end 51.415 56.958) (width 0.25) (layer B.Cu) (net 6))
 (segment (start 43.84499 48.99851) (end 44.66179 48.18171) (width 0.25) (layer B.Cu) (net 6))
 (segment (start 43.84499 52.77418) (end 43.84499 48.99851) (width 0.25) (layer B.Cu) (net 6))
 (segment (start 44.18182 53.11101) (end 43.84499 52.77418) (width 0.25) (layer B.Cu) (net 6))
 (segment (start 48.03001 53.11101) (end 44.18182 53.11101) (width 0.25) (layer B.Cu) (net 6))
 (segment (start 44.66179 48.18171) (end 45.495 47.3485) (width 0.25) (layer B.Cu) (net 6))
 (segment (start 51.321 56.402) (end 48.03001 53.11101) (width 0.25) (layer B.Cu) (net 6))
 (segment (start 51.321 57.052) (end 51.321 56.402) (width 0.25) (layer B.Cu) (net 6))
 (segment (start 61.37 44.098) (end 48.7455 44.098) (width 0.25) (layer B.Cu) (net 6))
 (segment (start 48.7455 44.098) (end 45.495 47.3485) (width 0.25) (layer B.Cu) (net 6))
 (segment (start 62.64 42.828) (end 61.37 44.098) (width 0.25) (layer B.Cu) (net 6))
 (segment (start 62.64 36.4775) (end 62.64 42.828) (width 0.25) (layer B.Cu) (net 6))
 (segment (start 55.6625 29.5) (end 62.64 36.4775) (width 0.25) (layer B.Cu) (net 6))
 (segment (start 31.955 56.958) (end 32.049 57.052) (width 0.25) (layer B.Cu) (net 7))
 (segment (start 21.619 56.958) (end 31.955 56.958) (width 0.25) (layer B.Cu) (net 7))
 (segment (start 39.97821 48.18171) (end 39.145 47.3485) (width 0.25) (layer B.Cu) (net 7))
 (segment (start 40.79501 52.77418) (end 40.79501 48.99851) (width 0.25) (layer B.Cu) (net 7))
 (segment (start 40.79501 48.99851) (end 39.97821 48.18171) (width 0.25) (layer B.Cu) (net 7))
 (segment (start 40.45818 53.11101) (end 40.79501 52.77418) (width 0.25) (layer B.Cu) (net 7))
 (segment (start 35.33999 53.11101) (end 40.45818 53.11101) (width 0.25) (layer B.Cu) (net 7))
 (segment (start 32.049 56.402) (end 35.33999 53.11101) (width 0.25) (layer B.Cu) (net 7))
 (segment (start 32.049 57.052) (end 32.049 56.402) (width 0.25) (layer B.Cu) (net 7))
 (segment (start 53.4695 42.193) (end 55.6625 40) (width 0.25) (layer B.Cu) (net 7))
 (segment (start 47.60052 42.193) (end 53.4695 42.193) (width 0.25) (layer B.Cu) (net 7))
 (segment (start 40.79501 48.99851) (end 47.60052 42.193) (width 0.25) (layer B.Cu) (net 7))
 (segment (start 21.619 51.558) (end 21.619 50.608) (width 0.25) (layer B.Cu) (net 8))
 (segment (start 31.8215 51.558) (end 32.16 51.8965) (width 0.25) (layer B.Cu) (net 8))
 (segment (start 21.619 51.558) (end 31.8215 51.558) (width 0.25) (layer B.Cu) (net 8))
 (segment (start 50.32199 52.77418) (end 50.32199 50.32001) (width 0.25) (layer B.Cu) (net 8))
 (segment (start 51.180811 53.633001) (end 50.32199 52.77418) (width 0.25) (layer B.Cu) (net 8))
 (segment (start 62.831003 53.633001) (end 51.180811 53.633001) (width 0.25) (layer B.Cu) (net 8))
 (segment (start 64.146001 54.947999) (end 62.831003 53.633001) (width 0.25) (layer B.Cu) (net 8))
 (segment (start 64.146001 58.968001) (end 64.146001 54.947999) (width 0.25) (layer B.Cu) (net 8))
 (segment (start 49.321 58.002) (end 50.352001 59.033001) (width 0.25) (layer B.Cu) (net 8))
 (segment (start 64.081001 59.033001) (end 64.146001 58.968001) (width 0.25) (layer B.Cu) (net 8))
 (segment (start 50.352001 59.033001) (end 64.081001 59.033001) (width 0.25) (layer B.Cu) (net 8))
 (segment (start 50.32199 50.32001) (end 50.702 49.94) (width 0.25) (layer B.Cu) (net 8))
 (segment (start 64.081001 49.482999) (end 69.879 55.280998) (width 0.25) (layer B.Cu) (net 8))
 (segment (start 55.604001 49.482999) (end 64.081001 49.482999) (width 0.25) (layer B.Cu) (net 8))
 (segment (start 55.147 49.94) (end 55.604001 49.482999) (width 0.25) (layer B.Cu) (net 8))
 (segment (start 50.702 49.94) (end 55.147 49.94) (width 0.25) (layer B.Cu) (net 8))
 (segment (start 69.879 57.941) (end 69.879 58.068) (width 0.25) (layer B.Cu) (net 8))
 (segment (start 69.879 55.280998) (end 69.879 57.941) (width 0.25) (layer B.Cu) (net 8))
 (segment (start 69.879 57.941) (end 67.535011 60.284989) (width 0.25) (layer B.Cu) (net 8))
 (segment (start 67.535011 60.284989) (end 21.810987 60.284989) (width 0.25) (layer B.Cu) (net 8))
 (segment (start 20.493999 58.968001) (end 20.493999 54.683001) (width 0.25) (layer B.Cu) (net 8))
 (segment (start 21.619 53.558) (end 21.619 51.558) (width 0.25) (layer B.Cu) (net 8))
 (segment (start 20.493999 54.683001) (end 21.619 53.558) (width 0.25) (layer B.Cu) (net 8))
 (segment (start 21.810987 60.284989) (end 20.493999 58.968001) (width 0.25) (layer B.Cu) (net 8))
 (segment (start 26 29.5) (end 33.46 29.5) (width 0.25) (layer B.Cu) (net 11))
 (segment (start 36 29.5) (end 43.46 29.5) (width 0.25) (layer B.Cu) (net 12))
 (segment (start 59.50429 28.66679) (end 60.3375 29.5) (width 0.25) (layer B.Cu) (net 9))
 (segment (start 58.68749 27.84999) (end 59.50429 28.66679) (width 0.25) (layer B.Cu) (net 9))
 (segment (start 48.80001 27.84999) (end 58.68749 27.84999) (width 0.25) (layer B.Cu) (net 9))
 (segment (start 47.15 29.5) (end 48.80001 27.84999) (width 0.25) (layer B.Cu) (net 9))
 (segment (start 46 29.5) (end 47.15 29.5) (width 0.25) (layer B.Cu) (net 9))
 (segment (start 31 39.5) (end 33.46 39.5) (width 0.25) (layer B.Cu) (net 13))
 (segment (start 36 39.5) (end 43.46 39.5) (width 0.25) (layer B.Cu) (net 1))
 (segment (start 46 39.5) (end 48.46 39.5) (width 0.25) (layer B.Cu) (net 2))
 (segment (start 58.68749 38.34999) (end 59.50429 39.16679) (width 0.25) (layer B.Cu) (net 10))
 (segment (start 52.15 39.5) (end 53.30001 38.34999) (width 0.25) (layer B.Cu) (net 10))
 (segment (start 59.50429 39.16679) (end 60.3375 40) (width 0.25) (layer B.Cu) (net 10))
 (segment (start 53.30001 38.34999) (end 58.68749 38.34999) (width 0.25) (layer B.Cu) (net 10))
 (segment (start 51 39.5) (end 52.15 39.5) (width 0.25) (layer B.Cu) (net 10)))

